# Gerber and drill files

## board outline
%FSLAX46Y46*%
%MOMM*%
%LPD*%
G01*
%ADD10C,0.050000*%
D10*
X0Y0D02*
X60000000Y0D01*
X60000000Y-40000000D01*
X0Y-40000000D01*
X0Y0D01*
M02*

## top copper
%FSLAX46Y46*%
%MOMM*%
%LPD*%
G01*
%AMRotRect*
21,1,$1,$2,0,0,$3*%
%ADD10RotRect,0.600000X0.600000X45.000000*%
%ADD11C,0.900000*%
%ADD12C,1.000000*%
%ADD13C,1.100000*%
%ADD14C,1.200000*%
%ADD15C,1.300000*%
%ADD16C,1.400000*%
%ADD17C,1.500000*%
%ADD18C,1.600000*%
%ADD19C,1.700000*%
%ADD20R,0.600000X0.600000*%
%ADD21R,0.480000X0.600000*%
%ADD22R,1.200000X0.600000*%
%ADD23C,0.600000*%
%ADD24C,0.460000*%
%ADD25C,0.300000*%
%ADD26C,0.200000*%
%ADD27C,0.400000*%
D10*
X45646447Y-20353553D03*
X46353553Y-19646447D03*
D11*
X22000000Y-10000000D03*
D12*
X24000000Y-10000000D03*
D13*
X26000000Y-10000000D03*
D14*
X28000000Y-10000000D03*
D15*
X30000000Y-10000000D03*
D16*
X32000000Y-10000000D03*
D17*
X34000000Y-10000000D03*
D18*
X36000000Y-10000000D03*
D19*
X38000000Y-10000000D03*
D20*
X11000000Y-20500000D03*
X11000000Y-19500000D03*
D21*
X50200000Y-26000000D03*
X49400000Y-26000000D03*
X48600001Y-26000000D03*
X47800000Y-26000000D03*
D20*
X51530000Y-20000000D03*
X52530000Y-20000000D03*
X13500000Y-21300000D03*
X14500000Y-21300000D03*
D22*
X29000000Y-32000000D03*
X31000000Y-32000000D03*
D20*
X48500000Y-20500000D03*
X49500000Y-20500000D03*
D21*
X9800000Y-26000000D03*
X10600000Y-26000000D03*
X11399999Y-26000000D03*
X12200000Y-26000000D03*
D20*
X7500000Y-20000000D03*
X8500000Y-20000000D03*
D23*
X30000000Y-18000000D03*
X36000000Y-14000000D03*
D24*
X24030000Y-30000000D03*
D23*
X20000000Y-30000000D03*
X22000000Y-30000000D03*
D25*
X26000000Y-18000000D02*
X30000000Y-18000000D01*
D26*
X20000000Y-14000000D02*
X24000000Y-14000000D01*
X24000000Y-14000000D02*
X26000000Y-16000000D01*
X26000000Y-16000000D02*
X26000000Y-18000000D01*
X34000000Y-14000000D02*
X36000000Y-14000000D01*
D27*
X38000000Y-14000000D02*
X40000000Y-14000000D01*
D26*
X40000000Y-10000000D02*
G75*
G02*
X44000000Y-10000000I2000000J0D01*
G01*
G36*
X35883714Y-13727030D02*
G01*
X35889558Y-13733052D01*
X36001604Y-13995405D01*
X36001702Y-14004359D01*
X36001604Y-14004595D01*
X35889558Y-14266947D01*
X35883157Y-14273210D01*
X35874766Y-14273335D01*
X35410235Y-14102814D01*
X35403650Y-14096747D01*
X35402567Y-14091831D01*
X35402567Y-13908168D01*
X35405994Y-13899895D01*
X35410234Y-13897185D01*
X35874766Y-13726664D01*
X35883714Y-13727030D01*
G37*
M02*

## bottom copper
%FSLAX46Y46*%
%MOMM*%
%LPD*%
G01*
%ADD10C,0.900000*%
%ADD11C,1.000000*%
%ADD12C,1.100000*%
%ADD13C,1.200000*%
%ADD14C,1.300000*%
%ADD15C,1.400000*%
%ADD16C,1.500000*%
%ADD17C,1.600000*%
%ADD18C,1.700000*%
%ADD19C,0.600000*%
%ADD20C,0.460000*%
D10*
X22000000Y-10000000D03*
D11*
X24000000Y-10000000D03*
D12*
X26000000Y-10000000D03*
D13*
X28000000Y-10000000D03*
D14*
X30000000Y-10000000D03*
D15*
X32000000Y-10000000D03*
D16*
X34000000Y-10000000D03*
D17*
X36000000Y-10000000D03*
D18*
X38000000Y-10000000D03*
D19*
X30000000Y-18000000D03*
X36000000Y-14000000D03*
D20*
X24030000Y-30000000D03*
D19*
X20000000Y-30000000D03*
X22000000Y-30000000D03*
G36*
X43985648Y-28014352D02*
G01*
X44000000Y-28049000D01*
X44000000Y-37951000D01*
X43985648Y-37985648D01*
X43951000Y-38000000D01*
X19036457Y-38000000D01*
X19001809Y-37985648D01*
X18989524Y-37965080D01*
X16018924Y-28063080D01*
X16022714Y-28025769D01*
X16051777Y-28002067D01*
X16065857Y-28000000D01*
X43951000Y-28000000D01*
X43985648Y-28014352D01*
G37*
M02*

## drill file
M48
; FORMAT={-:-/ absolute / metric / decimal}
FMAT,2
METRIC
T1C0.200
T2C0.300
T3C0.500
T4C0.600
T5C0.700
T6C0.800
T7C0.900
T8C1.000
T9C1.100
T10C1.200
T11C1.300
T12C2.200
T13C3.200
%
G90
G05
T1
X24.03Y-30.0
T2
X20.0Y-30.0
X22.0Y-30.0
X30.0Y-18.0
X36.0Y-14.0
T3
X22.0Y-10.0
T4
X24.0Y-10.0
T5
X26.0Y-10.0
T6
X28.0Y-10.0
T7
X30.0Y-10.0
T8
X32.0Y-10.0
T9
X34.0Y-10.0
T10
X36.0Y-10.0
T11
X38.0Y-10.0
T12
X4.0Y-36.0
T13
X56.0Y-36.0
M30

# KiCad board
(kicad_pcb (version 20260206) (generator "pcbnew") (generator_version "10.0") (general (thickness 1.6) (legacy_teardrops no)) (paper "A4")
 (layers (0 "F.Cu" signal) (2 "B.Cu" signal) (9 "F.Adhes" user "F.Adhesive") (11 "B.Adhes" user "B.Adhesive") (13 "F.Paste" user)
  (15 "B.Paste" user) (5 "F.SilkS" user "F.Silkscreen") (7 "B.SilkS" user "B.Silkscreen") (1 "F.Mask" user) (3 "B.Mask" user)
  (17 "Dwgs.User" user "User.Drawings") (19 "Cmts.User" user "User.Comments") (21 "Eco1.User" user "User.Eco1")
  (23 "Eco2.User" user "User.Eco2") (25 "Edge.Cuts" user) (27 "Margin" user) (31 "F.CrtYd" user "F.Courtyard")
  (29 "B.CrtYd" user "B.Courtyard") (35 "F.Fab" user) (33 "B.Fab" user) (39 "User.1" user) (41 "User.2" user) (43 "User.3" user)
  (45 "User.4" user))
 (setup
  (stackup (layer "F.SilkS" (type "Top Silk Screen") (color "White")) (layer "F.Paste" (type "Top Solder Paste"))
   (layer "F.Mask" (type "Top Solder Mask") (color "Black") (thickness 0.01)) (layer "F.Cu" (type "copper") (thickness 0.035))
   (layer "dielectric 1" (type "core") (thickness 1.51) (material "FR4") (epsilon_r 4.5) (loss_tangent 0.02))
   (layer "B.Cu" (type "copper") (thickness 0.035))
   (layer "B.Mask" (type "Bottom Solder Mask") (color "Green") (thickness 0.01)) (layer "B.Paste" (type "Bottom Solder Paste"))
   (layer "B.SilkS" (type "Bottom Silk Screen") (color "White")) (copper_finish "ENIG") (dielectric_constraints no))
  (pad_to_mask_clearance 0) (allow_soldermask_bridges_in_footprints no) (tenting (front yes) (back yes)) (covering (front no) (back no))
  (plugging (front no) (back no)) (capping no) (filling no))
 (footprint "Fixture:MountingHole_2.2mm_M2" (layer "F.Cu") (at 4 36)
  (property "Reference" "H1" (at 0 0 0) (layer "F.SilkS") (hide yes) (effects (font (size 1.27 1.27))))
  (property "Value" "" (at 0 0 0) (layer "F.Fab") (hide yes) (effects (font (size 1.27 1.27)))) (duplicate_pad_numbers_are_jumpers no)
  (pad "" np_thru_hole circle (at 0 0) (size 2.2 2.2) (drill 2.2) (layers "*.Cu" "*.Mask")))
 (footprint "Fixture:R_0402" (layer "F.Cu") (at 46 20 45)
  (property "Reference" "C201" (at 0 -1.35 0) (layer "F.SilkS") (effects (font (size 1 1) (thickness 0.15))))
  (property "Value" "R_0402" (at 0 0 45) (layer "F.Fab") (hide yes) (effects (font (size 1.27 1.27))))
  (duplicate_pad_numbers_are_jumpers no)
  (pad "1" smd rect (at -0.499999 0 45) (size 0.6 0.6) (layers "F.Cu" "F.Mask" "F.Paste") (thermal_bridge_angle 45))
  (pad "2" smd rect (at 0.499999 0 45) (size 0.6 0.6) (layers "F.Cu" "F.Mask" "F.Paste") (thermal_bridge_angle 45)))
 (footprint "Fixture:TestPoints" (layer "F.Cu") (at 30 10)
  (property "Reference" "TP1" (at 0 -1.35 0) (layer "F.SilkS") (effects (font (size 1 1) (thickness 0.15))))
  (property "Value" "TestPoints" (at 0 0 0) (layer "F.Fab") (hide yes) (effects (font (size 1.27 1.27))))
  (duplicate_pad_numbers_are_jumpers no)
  (pad "1" thru_hole circle (at -8 0) (size 0.9 0.9) (drill 0.5) (layers "*.Cu" "*.Mask") (remove_unused_layers no))
  (pad "2" thru_hole circle (at -6 0) (size 1 1) (drill 0.6) (layers "*.Cu" "*.Mask") (remove_unused_layers no))
  (pad "3" thru_hole circle (at -4 0) (size 1.1 1.1) (drill 0.7) (layers "*.Cu" "*.Mask") (remove_unused_layers no))
  (pad "4" thru_hole circle (at -2 0) (size 1.2 1.2) (drill 0.8) (layers "*.Cu" "*.Mask") (remove_unused_layers no))
  (pad "5" thru_hole circle (at 0 0) (size 1.3 1.3) (drill 0.9) (layers "*.Cu" "*.Mask") (remove_unused_layers no))
  (pad "6" thru_hole circle (at 2 0) (size 1.4 1.4) (drill 1) (layers "*.Cu" "*.Mask") (remove_unused_layers no))
  (pad "7" thru_hole circle (at 4 0) (size 1.5 1.5) (drill 1.1) (layers "*.Cu" "*.Mask") (remove_unused_layers no))
  (pad "8" thru_hole circle (at 6 0) (size 1.6 1.6) (drill 1.2) (layers "*.Cu" "*.Mask") (remove_unused_layers no))
  (pad "9" thru_hole circle (at 8 0) (size 1.7 1.7) (drill 1.3) (layers "*.Cu" "*.Mask") (remove_unused_layers no)))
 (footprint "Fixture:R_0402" (layer "F.Cu") (at 11 20 90)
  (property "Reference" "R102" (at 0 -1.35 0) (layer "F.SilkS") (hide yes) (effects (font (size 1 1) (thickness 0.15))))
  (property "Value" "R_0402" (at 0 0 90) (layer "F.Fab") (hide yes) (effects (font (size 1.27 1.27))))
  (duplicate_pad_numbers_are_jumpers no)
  (pad "1" smd rect (at -0.5 0 90) (size 0.6 0.6) (layers "F.Cu" "F.Mask" "F.Paste") (thermal_bridge_angle 45))
  (pad "2" smd rect (at 0.5 0 90) (size 0.6 0.6) (layers "F.Cu" "F.Mask" "F.Paste") (thermal_bridge_angle 45)))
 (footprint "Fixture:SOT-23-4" (layer "F.Cu") (at 49 26 180)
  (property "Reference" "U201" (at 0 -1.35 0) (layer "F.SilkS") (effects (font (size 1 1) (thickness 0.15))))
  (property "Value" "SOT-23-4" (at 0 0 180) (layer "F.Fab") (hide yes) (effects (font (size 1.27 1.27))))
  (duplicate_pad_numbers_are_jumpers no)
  (pad "1" smd rect (at -1.2 0 180) (size 0.48 0.6) (layers "F.Cu" "F.Mask" "F.Paste") (thermal_bridge_angle 45))
  (pad "2" smd rect (at -0.4 0 180) (size 0.48 0.6) (layers "F.Cu" "F.Mask" "F.Paste") (thermal_bridge_angle 45))
  (pad "3" smd rect (at 0.399999 0 180) (size 0.48 0.6) (layers "F.Cu" "F.Mask" "F.Paste") (thermal_bridge_angle 45))
  (pad "4" smd rect (at 1.2 0 180) (size 0.48 0.6) (layers "F.Cu" "F.Mask" "F.Paste") (thermal_bridge_angle 45)))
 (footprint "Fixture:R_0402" (layer "F.Cu") (at 52.03 20)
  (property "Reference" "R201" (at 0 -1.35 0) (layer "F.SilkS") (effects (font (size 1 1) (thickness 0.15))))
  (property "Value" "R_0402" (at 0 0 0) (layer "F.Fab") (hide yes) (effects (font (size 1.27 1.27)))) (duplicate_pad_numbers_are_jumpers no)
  (pad "1" smd rect (at -0.5 0) (size 0.6 0.6) (layers "F.Cu" "F.Mask" "F.Paste") (thermal_bridge_angle 45))
  (pad "2" smd rect (at 0.5 0) (size 0.6 0.6) (layers "F.Cu" "F.Mask" "F.Paste") (thermal_bridge_angle 45)))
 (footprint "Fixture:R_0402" (layer "F.Cu") (at 14 21.3)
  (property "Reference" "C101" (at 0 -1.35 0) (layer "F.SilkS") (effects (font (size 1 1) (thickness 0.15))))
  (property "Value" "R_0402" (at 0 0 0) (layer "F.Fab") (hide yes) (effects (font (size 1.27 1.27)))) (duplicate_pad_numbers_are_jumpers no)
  (pad "1" smd rect (at -0.5 0) (size 0.6 0.6) (layers "F.Cu" "F.Mask" "F.Paste") (thermal_bridge_angle 45))
  (pad "2" smd rect (at 0.5 0) (size 0.6 0.6) (layers "F.Cu" "F.Mask" "F.Paste") (thermal_bridge_angle 45)))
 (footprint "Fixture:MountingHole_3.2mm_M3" (layer "F.Cu") (at 56 36)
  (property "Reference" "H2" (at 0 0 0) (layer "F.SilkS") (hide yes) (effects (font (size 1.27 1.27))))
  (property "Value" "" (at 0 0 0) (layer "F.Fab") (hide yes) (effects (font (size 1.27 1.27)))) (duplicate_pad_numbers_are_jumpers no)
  (pad "" np_thru_hole circle (at 0 0) (size 3.2 3.2) (drill 3.2) (layers "*.Cu" "*.Mask")))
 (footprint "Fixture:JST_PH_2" (layer "F.Cu") (at 30 32)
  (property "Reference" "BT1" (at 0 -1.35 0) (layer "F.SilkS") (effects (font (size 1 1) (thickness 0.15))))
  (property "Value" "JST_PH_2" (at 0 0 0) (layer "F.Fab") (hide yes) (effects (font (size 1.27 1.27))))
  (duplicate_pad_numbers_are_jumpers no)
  (pad "1" smd rect (at -1 0) (size 1.2 0.6) (layers "F.Cu" "F.Mask" "F.Paste") (thermal_bridge_angle 45))
  (pad "2" smd rect (at 1 0) (size 1.2 0.6) (layers "F.Cu" "F.Mask" "F.Paste") (thermal_bridge_angle 45)))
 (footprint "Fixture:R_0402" (layer "F.Cu") (at 49 20.5)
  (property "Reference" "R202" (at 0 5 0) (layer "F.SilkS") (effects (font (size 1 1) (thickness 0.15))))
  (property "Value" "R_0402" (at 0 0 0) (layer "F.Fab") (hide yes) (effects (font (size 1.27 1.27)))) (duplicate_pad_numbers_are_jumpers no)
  (pad "1" smd rect (at -0.5 0) (size 0.6 0.6) (layers "F.Cu" "F.Mask" "F.Paste") (thermal_bridge_angle 45))
  (pad "2" smd rect (at 0.5 0) (size 0.6 0.6) (layers "F.Cu" "F.Mask" "F.Paste") (thermal_bridge_angle 45)))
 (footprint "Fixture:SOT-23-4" (layer "F.Cu") (at 11 26)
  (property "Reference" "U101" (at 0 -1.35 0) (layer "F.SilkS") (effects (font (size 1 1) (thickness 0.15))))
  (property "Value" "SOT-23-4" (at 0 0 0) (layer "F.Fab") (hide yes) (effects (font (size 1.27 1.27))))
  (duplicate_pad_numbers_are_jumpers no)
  (pad "1" smd rect (at -1.2 0) (size 0.48 0.6) (layers "F.Cu" "F.Mask" "F.Paste") (thermal_bridge_angle 45))
  (pad "2" smd rect (at -0.4 0) (size 0.48 0.6) (layers "F.Cu" "F.Mask" "F.Paste") (thermal_bridge_angle 45))
  (pad "3" smd rect (at 0.399999 0) (size 0.48 0.6) (layers "F.Cu" "F.Mask" "F.Paste") (thermal_bridge_angle 45))
  (pad "4" smd rect (at 1.2 0) (size 0.48 0.6) (layers "F.Cu" "F.Mask" "F.Paste") (thermal_bridge_angle 45)))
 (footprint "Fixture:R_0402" (layer "F.Cu") (at 8 20)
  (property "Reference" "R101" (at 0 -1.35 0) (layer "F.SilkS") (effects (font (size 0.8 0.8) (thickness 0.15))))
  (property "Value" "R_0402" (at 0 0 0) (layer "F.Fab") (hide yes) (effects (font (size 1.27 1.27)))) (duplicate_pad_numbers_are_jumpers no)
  (pad "1" smd rect (at -0.5 0) (size 0.6 0.6) (layers "F.Cu" "F.Mask" "F.Paste") (thermal_bridge_angle 45))
  (pad "2" smd rect (at 0.5 0) (size 0.6 0.6) (layers "F.Cu" "F.Mask" "F.Paste") (thermal_bridge_angle 45)))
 (gr_rect (start 0 0) (end 60 40) (stroke (width 0.05) (type default)) (fill no) (layer "Edge.Cuts"))
 (segment (start 26 18) (end 30 18) (width 0.3) (layer "F.Cu") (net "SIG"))
 (segment (start 20 14) (end 24 14) (width 0.2) (layer "F.Cu") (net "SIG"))
 (segment (start 24 14) (end 26 16) (width 0.2) (layer "F.Cu") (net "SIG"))
 (segment (start 26 16) (end 26 18) (width 0.2) (layer "F.Cu") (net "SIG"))
 (via (at 30 18) (size 0.6) (drill 0.3) (layers "F.Cu" "B.Cu") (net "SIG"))
 (segment (start 34 14) (end 36 14) (width 0.2) (layer "F.Cu") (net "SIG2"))
 (via (at 36 14) (size 0.6) (drill 0.3) (layers "F.Cu" "B.Cu")
  (teardrops (best_length_ratio 0.5) (max_length 1) (best_width_ratio 1) (max_width 2) (curved_edges no) (filter_ratio 0.9) (enabled yes)
   (allow_two_segments yes) (prefer_zone_connections yes))
  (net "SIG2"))
 (segment (start 38 14) (end 40 14) (width 0.4) (layer "F.Cu") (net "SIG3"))
 (arc (start 40 10) (mid 42 8) (end 44 10) (width 0.2) (layer "F.Cu") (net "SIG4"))
 (via (at 24.03 30) (size 0.46) (drill 0.2) (layers "F.Cu" "B.Cu") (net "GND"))
 (via (at 20 30) (size 0.6) (drill 0.3) (layers "F.Cu" "B.Cu") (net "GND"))
 (via (at 22 30) (size 0.6) (drill 0.3) (layers "F.Cu" "B.Cu") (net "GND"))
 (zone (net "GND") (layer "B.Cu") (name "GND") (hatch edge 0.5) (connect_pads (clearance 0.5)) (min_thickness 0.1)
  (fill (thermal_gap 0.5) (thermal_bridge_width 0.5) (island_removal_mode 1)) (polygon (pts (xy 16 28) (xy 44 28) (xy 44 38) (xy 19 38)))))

